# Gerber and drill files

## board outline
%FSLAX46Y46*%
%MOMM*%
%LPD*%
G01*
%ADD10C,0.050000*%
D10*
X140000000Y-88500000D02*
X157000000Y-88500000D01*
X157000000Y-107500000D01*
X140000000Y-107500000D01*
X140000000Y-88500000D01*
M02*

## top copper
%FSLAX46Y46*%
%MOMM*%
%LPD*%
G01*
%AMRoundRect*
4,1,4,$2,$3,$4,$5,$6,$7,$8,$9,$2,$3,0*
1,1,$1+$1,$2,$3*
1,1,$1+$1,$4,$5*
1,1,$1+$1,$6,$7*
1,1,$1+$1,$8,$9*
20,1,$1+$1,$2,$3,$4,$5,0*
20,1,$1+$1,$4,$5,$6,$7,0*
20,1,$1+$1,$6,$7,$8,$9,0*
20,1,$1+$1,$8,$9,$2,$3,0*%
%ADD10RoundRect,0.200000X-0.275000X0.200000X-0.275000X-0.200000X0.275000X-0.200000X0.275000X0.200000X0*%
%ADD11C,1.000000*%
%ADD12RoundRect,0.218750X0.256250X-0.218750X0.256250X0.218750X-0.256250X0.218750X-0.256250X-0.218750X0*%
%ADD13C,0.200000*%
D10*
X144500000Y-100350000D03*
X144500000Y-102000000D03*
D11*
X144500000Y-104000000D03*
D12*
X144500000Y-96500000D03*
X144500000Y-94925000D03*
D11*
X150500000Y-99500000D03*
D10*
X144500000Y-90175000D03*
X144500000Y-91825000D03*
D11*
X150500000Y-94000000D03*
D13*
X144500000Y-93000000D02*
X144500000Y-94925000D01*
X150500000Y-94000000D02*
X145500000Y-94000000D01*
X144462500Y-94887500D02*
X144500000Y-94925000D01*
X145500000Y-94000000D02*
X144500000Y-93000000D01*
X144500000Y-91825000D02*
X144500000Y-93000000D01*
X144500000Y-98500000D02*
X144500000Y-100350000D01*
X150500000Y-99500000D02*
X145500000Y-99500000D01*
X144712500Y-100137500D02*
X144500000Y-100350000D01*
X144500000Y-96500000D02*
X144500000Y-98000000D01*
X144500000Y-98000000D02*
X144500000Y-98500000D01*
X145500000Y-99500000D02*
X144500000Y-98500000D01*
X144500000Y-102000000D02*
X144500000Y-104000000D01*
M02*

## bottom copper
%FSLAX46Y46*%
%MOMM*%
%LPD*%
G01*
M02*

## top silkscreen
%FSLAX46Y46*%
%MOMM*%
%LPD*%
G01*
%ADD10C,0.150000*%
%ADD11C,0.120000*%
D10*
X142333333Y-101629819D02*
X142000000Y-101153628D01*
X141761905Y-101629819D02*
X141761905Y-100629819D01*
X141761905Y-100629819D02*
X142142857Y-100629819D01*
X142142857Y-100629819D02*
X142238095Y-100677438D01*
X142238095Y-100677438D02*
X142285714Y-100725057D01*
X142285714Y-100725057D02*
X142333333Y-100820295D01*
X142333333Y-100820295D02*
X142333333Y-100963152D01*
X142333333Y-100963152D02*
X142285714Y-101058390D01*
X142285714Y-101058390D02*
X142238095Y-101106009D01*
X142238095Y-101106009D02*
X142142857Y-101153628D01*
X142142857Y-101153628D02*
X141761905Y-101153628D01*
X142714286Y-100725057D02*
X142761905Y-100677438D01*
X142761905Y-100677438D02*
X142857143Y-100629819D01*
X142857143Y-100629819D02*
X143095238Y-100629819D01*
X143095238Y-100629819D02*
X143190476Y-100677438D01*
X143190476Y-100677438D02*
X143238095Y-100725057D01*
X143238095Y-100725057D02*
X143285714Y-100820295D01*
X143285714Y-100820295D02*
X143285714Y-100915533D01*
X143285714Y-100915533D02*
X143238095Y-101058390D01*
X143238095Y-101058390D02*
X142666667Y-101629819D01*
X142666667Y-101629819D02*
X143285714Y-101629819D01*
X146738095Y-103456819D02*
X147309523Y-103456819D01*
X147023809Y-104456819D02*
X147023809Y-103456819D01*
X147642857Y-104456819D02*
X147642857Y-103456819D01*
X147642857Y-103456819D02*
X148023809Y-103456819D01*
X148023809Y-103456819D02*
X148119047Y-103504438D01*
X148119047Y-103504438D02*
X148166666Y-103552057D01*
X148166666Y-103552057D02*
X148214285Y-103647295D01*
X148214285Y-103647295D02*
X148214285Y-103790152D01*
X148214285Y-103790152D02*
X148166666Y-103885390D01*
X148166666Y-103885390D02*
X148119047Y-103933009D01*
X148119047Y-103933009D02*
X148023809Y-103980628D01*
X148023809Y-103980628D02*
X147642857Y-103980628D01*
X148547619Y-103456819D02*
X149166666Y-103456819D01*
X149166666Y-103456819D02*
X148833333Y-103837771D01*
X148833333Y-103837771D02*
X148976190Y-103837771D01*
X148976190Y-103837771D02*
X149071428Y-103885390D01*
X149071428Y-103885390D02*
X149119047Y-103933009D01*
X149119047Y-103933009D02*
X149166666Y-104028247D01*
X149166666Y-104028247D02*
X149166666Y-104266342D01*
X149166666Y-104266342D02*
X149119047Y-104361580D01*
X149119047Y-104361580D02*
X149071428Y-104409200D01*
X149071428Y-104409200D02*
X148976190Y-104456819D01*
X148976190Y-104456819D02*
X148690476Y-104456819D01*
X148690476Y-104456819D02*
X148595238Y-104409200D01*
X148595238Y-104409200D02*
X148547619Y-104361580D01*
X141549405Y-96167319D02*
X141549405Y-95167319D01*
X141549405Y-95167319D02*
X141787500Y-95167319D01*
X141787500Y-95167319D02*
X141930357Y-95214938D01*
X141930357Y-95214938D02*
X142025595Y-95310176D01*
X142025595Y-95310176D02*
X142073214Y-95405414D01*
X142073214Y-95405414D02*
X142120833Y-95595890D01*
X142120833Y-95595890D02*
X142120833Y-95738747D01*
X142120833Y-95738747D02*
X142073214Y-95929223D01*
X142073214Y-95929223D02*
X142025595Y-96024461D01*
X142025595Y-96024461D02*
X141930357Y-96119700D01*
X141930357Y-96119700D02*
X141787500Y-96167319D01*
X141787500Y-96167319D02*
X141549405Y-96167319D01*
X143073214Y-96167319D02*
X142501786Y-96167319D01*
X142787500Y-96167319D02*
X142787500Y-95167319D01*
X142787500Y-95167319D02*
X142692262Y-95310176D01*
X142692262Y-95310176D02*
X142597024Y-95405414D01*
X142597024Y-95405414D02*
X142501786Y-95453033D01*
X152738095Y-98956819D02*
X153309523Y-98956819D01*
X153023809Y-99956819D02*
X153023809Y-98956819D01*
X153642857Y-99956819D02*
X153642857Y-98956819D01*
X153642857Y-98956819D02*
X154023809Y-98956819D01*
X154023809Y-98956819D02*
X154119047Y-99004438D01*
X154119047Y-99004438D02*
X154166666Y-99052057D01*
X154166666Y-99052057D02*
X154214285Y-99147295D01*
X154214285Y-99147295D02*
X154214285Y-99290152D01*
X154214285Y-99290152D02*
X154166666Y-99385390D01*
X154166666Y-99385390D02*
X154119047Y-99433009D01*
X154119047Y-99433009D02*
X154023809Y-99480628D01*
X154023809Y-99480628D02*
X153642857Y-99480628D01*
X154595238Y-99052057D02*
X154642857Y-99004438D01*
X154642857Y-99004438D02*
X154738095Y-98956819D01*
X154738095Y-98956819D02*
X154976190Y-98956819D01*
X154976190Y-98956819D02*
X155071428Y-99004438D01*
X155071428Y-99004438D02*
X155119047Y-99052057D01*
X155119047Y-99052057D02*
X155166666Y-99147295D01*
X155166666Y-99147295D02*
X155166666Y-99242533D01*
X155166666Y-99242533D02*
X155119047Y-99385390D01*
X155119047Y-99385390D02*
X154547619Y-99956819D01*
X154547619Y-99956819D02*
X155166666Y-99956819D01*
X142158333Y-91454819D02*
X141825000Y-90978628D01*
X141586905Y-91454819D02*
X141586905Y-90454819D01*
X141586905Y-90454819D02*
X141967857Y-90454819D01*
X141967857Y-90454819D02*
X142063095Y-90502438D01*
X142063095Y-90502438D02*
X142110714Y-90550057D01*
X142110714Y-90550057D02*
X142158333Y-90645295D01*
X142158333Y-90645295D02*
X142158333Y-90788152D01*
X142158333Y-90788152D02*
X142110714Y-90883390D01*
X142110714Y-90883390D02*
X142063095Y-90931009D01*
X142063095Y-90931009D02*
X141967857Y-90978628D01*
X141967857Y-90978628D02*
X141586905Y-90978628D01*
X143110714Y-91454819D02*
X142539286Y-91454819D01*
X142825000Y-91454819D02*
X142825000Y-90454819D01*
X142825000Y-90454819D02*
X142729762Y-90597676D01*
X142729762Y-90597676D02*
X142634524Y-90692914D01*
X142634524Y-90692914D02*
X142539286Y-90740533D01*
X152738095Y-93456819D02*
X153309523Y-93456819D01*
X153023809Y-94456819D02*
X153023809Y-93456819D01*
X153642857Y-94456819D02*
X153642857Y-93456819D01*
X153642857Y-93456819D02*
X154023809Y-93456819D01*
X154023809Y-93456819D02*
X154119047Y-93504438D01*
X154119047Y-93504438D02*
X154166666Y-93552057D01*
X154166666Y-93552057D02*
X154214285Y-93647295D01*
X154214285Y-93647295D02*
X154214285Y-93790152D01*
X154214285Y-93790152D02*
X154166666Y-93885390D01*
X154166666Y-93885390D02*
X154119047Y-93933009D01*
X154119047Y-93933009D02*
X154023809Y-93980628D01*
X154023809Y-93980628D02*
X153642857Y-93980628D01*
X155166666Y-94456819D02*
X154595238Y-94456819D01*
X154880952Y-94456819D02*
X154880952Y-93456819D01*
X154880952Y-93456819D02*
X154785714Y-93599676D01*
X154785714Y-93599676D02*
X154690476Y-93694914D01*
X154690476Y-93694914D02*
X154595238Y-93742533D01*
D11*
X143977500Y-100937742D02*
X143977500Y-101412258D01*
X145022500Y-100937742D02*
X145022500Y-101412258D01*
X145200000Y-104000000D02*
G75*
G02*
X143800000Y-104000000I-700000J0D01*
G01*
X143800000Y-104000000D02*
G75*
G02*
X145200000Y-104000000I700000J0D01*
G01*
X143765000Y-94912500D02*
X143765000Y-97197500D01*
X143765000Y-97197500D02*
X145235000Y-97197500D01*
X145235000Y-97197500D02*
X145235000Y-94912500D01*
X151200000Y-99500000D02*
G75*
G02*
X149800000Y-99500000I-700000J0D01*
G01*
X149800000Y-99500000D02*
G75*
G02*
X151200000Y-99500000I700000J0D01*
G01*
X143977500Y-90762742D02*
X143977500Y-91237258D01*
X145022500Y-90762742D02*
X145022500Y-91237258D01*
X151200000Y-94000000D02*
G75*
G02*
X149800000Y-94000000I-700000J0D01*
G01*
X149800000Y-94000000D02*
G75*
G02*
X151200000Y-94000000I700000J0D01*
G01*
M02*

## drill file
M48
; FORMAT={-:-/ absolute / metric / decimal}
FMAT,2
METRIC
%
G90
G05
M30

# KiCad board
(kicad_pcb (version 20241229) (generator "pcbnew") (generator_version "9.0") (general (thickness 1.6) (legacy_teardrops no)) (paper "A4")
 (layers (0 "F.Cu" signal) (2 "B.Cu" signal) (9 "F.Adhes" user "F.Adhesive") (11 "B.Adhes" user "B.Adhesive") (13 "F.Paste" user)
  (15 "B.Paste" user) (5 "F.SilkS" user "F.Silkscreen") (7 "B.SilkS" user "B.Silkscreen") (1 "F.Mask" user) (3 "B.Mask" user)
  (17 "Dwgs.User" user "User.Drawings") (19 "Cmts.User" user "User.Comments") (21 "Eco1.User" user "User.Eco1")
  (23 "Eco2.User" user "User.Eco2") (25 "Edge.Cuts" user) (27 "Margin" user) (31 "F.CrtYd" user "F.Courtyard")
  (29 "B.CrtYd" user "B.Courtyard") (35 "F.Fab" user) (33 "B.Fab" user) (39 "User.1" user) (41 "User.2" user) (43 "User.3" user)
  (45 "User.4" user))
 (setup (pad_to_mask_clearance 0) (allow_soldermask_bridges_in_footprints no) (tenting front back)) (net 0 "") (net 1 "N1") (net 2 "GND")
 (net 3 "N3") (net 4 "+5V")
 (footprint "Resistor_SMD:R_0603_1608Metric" (layer "F.Cu") (at 144.5 101.175 -90)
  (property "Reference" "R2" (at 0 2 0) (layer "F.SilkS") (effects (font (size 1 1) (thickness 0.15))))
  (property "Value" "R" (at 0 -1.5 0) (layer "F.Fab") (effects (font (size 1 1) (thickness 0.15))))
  (fp_line (start -0.237258 0.5225) (end 0.237258 0.5225) (stroke (width 0.12) (type solid)) (layer "F.SilkS"))
  (fp_line (start -0.237258 -0.5225) (end 0.237258 -0.5225) (stroke (width 0.12) (type solid)) (layer "F.SilkS"))
  (pad "1" smd roundrect (at -0.825 0 270) (size 0.8 0.95) (layers "F.Cu" "F.Mask" "F.Paste") (roundrect_rratio 0.25) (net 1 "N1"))
  (pad "2" smd roundrect (at 0.825 0 270) (size 0.8 0.95) (layers "F.Cu" "F.Mask" "F.Paste") (roundrect_rratio 0.25) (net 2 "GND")))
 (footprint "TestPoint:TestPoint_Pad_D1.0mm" (layer "F.Cu") (at 144.5 104)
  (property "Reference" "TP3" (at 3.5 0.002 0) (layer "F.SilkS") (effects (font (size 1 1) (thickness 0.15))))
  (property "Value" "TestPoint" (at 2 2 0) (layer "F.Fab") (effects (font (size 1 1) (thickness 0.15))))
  (fp_circle (center 0 0) (end 0 0.7) (stroke (width 0.12) (type solid)) (fill no) (layer "F.SilkS"))
  (pad "1" smd circle (at 0 0) (size 1 1) (layers "F.Cu" "F.Mask") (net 2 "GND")))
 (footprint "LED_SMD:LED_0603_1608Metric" (layer "F.Cu") (at 144.5 95.7125 90)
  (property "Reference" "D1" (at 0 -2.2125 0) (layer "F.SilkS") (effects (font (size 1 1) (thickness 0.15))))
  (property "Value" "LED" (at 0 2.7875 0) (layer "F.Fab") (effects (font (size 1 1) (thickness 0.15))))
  (fp_line (start 0.8 -0.735) (end -1.485 -0.735) (stroke (width 0.12) (type solid)) (layer "F.SilkS"))
  (fp_line (start -1.485 -0.735) (end -1.485 0.735) (stroke (width 0.12) (type solid)) (layer "F.SilkS"))
  (fp_line (start -1.485 0.735) (end 0.8 0.735) (stroke (width 0.12) (type solid)) (layer "F.SilkS"))
  (pad "1" smd roundrect (at -0.7875 0 90) (size 0.875 0.95) (layers "F.Cu" "F.Mask" "F.Paste") (roundrect_rratio 0.25) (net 1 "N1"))
  (pad "2" smd roundrect (at 0.7875 0 90) (size 0.875 0.95) (layers "F.Cu" "F.Mask" "F.Paste") (roundrect_rratio 0.25) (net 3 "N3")))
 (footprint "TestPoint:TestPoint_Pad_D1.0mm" (layer "F.Cu") (at 150.5 99.5)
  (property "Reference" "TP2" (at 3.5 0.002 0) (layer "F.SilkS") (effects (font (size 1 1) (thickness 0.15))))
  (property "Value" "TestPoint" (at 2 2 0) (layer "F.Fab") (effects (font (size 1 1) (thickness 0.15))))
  (fp_circle (center 0 0) (end 0 0.7) (stroke (width 0.12) (type solid)) (fill no) (layer "F.SilkS"))
  (pad "1" smd circle (at 0 0) (size 1 1) (layers "F.Cu" "F.Mask") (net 1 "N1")))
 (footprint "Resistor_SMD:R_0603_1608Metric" (layer "F.Cu") (at 144.5 91 -90)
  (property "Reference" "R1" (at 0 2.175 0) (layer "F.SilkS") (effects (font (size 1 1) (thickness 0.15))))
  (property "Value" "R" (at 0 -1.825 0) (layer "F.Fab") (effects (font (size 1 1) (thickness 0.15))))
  (fp_line (start -0.237258 0.5225) (end 0.237258 0.5225) (stroke (width 0.12) (type solid)) (layer "F.SilkS"))
  (fp_line (start -0.237258 -0.5225) (end 0.237258 -0.5225) (stroke (width 0.12) (type solid)) (layer "F.SilkS"))
  (pad "1" smd roundrect (at -0.825 0 270) (size 0.8 0.95) (layers "F.Cu" "F.Mask" "F.Paste") (roundrect_rratio 0.25) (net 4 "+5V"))
  (pad "2" smd roundrect (at 0.825 0 270) (size 0.8 0.95) (layers "F.Cu" "F.Mask" "F.Paste") (roundrect_rratio 0.25) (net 3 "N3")))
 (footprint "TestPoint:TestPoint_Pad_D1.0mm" (layer "F.Cu") (at 150.5 94)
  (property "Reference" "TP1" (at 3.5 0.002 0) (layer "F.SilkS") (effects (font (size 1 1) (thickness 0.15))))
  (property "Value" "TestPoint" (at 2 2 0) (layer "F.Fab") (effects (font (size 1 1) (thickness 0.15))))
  (fp_circle (center 0 0) (end 0 0.7) (stroke (width 0.12) (type solid)) (fill no) (layer "F.SilkS"))
  (pad "1" smd circle (at 0 0) (size 1 1) (layers "F.Cu" "F.Mask") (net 3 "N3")))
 (gr_rect (start 140 88.5) (end 157 107.5) (stroke (width 0.05) (type default)) (fill no) (layer "Edge.Cuts"))
 (segment (start 144.5 93) (end 144.5 94.925) (width 0.2) (layer "F.Cu") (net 3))
 (segment (start 150.5 94) (end 145.5 94) (width 0.2) (layer "F.Cu") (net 3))
 (segment (start 144.4625 94.8875) (end 144.5 94.925) (width 0.2) (layer "F.Cu") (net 3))
 (segment (start 145.5 94) (end 144.5 93) (width 0.2) (layer "F.Cu") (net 3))
 (segment (start 144.5 91.825) (end 144.5 93) (width 0.2) (layer "F.Cu") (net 3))
 (segment (start 144.5 98.5) (end 144.5 100.35) (width 0.2) (layer "F.Cu") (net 1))
 (segment (start 150.5 99.5) (end 145.5 99.5) (width 0.2) (layer "F.Cu") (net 1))
 (segment (start 144.7125 100.1375) (end 144.5 100.35) (width 0.2) (layer "F.Cu") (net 1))
 (segment (start 144.5 96.5) (end 144.5 98) (width 0.2) (layer "F.Cu") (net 1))
 (segment (start 144.5 98) (end 144.5 98.5) (width 0.2) (layer "F.Cu") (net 1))
 (segment (start 145.5 99.5) (end 144.5 98.5) (width 0.2) (layer "F.Cu") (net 1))
 (segment (start 144.5 102) (end 144.5 104) (width 0.2) (layer "F.Cu") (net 2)))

